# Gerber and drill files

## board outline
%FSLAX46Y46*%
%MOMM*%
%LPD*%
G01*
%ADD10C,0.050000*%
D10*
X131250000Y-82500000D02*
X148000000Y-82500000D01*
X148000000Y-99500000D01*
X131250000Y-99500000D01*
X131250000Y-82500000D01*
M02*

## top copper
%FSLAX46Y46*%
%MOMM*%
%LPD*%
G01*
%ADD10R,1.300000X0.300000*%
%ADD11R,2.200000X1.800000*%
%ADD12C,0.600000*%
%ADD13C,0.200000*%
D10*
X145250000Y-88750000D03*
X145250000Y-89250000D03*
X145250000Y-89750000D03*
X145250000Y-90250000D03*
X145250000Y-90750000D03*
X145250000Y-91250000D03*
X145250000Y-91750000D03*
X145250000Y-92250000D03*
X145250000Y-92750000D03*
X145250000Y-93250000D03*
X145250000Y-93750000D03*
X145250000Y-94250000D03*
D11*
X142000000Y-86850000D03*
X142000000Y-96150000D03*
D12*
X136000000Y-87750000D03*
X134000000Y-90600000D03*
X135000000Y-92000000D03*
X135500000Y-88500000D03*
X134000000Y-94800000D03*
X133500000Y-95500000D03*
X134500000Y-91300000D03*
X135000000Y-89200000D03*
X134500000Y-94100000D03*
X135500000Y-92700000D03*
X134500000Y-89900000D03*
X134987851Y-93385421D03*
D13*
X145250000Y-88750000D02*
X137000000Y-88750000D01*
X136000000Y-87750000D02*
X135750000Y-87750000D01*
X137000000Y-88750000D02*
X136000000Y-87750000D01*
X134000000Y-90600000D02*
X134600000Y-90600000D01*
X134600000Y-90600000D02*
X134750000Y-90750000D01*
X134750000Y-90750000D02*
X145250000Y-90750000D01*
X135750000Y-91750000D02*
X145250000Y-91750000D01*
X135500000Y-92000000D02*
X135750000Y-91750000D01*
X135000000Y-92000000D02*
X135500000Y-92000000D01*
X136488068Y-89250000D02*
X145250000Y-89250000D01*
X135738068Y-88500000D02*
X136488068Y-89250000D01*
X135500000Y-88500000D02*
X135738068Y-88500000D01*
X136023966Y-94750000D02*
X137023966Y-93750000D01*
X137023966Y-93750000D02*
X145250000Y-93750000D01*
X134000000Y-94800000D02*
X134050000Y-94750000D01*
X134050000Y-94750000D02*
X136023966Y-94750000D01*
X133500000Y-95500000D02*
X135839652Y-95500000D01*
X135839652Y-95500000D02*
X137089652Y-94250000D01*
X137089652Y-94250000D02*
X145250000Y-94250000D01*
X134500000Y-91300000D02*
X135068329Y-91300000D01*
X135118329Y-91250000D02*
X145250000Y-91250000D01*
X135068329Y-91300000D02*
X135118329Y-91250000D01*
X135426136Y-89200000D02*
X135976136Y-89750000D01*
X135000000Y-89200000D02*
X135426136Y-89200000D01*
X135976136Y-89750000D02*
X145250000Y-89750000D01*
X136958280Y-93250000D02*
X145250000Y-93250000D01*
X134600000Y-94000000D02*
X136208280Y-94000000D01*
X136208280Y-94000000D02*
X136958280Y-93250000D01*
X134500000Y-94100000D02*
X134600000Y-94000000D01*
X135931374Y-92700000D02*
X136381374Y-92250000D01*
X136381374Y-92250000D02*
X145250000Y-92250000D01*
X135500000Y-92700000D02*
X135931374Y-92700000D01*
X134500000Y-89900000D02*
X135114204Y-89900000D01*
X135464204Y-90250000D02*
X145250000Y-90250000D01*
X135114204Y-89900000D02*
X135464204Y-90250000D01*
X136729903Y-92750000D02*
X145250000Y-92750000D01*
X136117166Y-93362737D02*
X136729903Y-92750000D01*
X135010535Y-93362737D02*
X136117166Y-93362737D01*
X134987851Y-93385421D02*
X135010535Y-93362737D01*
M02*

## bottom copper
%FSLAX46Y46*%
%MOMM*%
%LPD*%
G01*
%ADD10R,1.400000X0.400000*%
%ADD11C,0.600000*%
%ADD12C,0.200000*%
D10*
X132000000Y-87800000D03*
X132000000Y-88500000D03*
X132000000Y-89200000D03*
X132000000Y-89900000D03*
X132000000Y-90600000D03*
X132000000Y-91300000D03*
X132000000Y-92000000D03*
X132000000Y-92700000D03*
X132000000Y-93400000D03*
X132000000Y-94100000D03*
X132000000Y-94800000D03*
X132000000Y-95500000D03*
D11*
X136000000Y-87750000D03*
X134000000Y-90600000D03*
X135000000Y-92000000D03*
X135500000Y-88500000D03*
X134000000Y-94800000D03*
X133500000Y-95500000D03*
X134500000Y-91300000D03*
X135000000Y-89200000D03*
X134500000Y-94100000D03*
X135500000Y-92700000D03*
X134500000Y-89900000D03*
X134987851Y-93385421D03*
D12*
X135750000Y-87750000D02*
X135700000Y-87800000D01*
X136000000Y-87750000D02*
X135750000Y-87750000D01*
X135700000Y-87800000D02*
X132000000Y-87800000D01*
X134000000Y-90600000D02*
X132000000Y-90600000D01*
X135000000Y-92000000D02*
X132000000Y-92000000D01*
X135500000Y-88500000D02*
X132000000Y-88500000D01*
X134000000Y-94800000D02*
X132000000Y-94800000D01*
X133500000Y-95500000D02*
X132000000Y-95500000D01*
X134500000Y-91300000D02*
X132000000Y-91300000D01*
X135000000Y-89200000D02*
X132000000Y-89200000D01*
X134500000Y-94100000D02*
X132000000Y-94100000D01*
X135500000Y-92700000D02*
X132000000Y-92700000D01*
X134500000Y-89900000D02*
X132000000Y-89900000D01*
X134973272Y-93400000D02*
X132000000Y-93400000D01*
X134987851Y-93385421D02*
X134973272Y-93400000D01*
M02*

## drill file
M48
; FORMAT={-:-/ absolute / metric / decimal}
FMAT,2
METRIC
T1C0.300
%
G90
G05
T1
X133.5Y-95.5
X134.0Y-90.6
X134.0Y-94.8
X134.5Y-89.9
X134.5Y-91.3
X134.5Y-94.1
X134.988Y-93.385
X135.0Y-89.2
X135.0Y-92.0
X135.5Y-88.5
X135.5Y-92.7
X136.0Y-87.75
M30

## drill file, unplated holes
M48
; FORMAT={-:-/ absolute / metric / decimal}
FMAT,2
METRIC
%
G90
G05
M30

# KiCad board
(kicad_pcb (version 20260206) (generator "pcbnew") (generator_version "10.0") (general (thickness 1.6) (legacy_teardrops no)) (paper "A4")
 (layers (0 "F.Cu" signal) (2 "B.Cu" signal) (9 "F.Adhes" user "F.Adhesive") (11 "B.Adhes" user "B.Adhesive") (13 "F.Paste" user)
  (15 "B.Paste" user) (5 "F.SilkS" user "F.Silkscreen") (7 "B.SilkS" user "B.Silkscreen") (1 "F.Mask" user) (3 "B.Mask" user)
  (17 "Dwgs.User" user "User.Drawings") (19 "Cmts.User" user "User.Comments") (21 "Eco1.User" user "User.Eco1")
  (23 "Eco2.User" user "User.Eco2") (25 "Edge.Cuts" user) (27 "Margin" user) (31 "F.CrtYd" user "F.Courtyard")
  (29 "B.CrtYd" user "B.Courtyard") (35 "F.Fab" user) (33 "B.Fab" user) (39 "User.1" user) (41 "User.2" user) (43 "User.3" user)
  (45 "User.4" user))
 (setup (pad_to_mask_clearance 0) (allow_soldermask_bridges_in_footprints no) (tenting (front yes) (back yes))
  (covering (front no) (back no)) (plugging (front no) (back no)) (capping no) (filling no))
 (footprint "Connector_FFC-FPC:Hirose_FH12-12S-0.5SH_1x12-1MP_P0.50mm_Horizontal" (layer "F.Cu") (at 143.4 91.5 -90)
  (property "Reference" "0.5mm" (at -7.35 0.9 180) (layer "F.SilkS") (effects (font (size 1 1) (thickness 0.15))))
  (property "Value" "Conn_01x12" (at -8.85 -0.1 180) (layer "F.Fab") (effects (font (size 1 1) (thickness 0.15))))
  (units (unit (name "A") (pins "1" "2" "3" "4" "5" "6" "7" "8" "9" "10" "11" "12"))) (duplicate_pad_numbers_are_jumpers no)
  (pad "1" smd rect (at -2.75 -1.85 270) (size 0.3 1.3) (layers "F.Cu" "F.Mask" "F.Paste") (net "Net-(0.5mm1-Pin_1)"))
  (pad "2" smd rect (at -2.25 -1.85 270) (size 0.3 1.3) (layers "F.Cu" "F.Mask" "F.Paste") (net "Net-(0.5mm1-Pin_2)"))
  (pad "3" smd rect (at -1.75 -1.85 270) (size 0.3 1.3) (layers "F.Cu" "F.Mask" "F.Paste") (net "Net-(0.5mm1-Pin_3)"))
  (pad "4" smd rect (at -1.25 -1.85 270) (size 0.3 1.3) (layers "F.Cu" "F.Mask" "F.Paste") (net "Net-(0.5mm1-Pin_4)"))
  (pad "5" smd rect (at -0.75 -1.85 270) (size 0.3 1.3) (layers "F.Cu" "F.Mask" "F.Paste") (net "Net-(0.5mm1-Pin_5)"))
  (pad "6" smd rect (at -0.25 -1.85 270) (size 0.3 1.3) (layers "F.Cu" "F.Mask" "F.Paste") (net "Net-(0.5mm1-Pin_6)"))
  (pad "7" smd rect (at 0.25 -1.85 270) (size 0.3 1.3) (layers "F.Cu" "F.Mask" "F.Paste") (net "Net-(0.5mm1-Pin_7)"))
  (pad "8" smd rect (at 0.75 -1.85 270) (size 0.3 1.3) (layers "F.Cu" "F.Mask" "F.Paste") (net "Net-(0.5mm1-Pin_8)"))
  (pad "9" smd rect (at 1.25 -1.85 270) (size 0.3 1.3) (layers "F.Cu" "F.Mask" "F.Paste") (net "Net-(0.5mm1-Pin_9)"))
  (pad "10" smd rect (at 1.75 -1.85 270) (size 0.3 1.3) (layers "F.Cu" "F.Mask" "F.Paste") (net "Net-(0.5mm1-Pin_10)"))
  (pad "11" smd rect (at 2.25 -1.85 270) (size 0.3 1.3) (layers "F.Cu" "F.Mask" "F.Paste") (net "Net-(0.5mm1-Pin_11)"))
  (pad "12" smd rect (at 2.75 -1.85 270) (size 0.3 1.3) (layers "F.Cu" "F.Mask" "F.Paste") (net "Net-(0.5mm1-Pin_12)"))
  (pad "MP" smd rect (at -4.65 1.4 270) (size 1.8 2.2) (layers "F.Cu" "F.Mask" "F.Paste"))
  (pad "MP" smd rect (at 4.65 1.4 270) (size 1.8 2.2) (layers "F.Cu" "F.Mask" "F.Paste")))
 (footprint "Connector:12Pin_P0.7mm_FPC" (layer "B.Cu") (at 132 91.65 -90)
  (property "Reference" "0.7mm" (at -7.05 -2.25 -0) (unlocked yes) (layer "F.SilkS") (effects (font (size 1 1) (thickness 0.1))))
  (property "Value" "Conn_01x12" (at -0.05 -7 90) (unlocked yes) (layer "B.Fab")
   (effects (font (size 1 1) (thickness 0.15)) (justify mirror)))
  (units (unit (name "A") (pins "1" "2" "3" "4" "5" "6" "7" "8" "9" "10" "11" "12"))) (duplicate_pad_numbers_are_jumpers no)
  (pad "1" connect rect (at -3.85 0 270) (size 0.4 1.4) (layers "B.Cu" "B.Mask") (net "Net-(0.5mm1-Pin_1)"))
  (pad "2" connect rect (at -3.15 0 270) (size 0.4 1.4) (layers "B.Cu" "B.Mask") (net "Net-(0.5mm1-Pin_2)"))
  (pad "3" connect rect (at -2.45 0 270) (size 0.4 1.4) (layers "B.Cu" "B.Mask") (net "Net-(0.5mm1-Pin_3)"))
  (pad "4" connect rect (at -1.75 0 270) (size 0.4 1.4) (layers "B.Cu" "B.Mask") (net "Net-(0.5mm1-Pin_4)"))
  (pad "5" connect rect (at -1.05 0 270) (size 0.4 1.4) (layers "B.Cu" "B.Mask") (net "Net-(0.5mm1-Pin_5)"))
  (pad "6" connect rect (at -0.35 0 270) (size 0.4 1.4) (layers "B.Cu" "B.Mask") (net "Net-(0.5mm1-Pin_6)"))
  (pad "7" connect rect (at 0.35 0 270) (size 0.4 1.4) (layers "B.Cu" "B.Mask") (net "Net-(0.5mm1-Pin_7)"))
  (pad "8" connect rect (at 1.05 0 270) (size 0.4 1.4) (layers "B.Cu" "B.Mask") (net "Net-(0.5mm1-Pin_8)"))
  (pad "9" connect rect (at 1.75 0 270) (size 0.4 1.4) (layers "B.Cu" "B.Mask") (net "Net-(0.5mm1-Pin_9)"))
  (pad "10" connect rect (at 2.45 0 270) (size 0.4 1.4) (layers "B.Cu" "B.Mask") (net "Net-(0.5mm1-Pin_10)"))
  (pad "11" connect rect (at 3.15 0 270) (size 0.4 1.4) (layers "B.Cu" "B.Mask") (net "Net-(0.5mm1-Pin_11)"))
  (pad "12" connect rect (at 3.85 0 270) (size 0.4 1.4) (layers "B.Cu" "B.Mask") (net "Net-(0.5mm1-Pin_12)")))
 (gr_rect (start 131.25 82.5) (end 148 99.5) (stroke (width 0.05) (type default)) (fill no) (layer "Edge.Cuts"))
 (segment (start 145.25 88.75) (end 137 88.75) (width 0.2) (layer "F.Cu") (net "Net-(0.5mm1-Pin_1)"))
 (segment (start 136 87.75) (end 135.75 87.75) (width 0.2) (layer "F.Cu") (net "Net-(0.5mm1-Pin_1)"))
 (segment (start 137 88.75) (end 136 87.75) (width 0.2) (layer "F.Cu") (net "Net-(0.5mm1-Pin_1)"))
 (via (at 136 87.75) (size 0.6) (drill 0.3) (layers "F.Cu" "B.Cu") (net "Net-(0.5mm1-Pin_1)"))
 (segment (start 135.75 87.75) (end 135.7 87.8) (width 0.2) (layer "B.Cu") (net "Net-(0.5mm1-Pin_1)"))
 (segment (start 136 87.75) (end 135.75 87.75) (width 0.2) (layer "B.Cu") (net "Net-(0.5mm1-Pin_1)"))
 (segment (start 135.7 87.8) (end 132 87.8) (width 0.2) (layer "B.Cu") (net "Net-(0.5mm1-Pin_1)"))
 (segment (start 134 90.6) (end 134.6 90.6) (width 0.2) (layer "F.Cu") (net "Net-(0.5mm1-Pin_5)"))
 (segment (start 134.6 90.6) (end 134.75 90.75) (width 0.2) (layer "F.Cu") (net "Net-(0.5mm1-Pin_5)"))
 (segment (start 134.75 90.75) (end 145.25 90.75) (width 0.2) (layer "F.Cu") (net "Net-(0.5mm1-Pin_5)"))
 (via (at 134 90.6) (size 0.6) (drill 0.3) (layers "F.Cu" "B.Cu") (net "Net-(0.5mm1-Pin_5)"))
 (segment (start 134 90.6) (end 132 90.6) (width 0.2) (layer "B.Cu") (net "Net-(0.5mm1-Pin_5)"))
 (segment (start 135.75 91.75) (end 145.25 91.75) (width 0.2) (layer "F.Cu") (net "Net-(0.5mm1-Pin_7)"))
 (segment (start 135.5 92) (end 135.75 91.75) (width 0.2) (layer "F.Cu") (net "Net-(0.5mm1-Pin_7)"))
 (segment (start 135 92) (end 135.5 92) (width 0.2) (layer "F.Cu") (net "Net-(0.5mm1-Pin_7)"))
 (via (at 135 92) (size 0.6) (drill 0.3) (layers "F.Cu" "B.Cu") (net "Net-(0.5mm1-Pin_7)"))
 (segment (start 135 92) (end 132 92) (width 0.2) (layer "B.Cu") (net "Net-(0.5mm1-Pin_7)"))
 (segment (start 136.488068 89.25) (end 145.25 89.25) (width 0.2) (layer "F.Cu") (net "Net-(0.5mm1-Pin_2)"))
 (segment (start 135.738068 88.5) (end 136.488068 89.25) (width 0.2) (layer "F.Cu") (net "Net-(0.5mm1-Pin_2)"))
 (segment (start 135.5 88.5) (end 135.738068 88.5) (width 0.2) (layer "F.Cu") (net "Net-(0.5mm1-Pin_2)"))
 (via (at 135.5 88.5) (size 0.6) (drill 0.3) (layers "F.Cu" "B.Cu") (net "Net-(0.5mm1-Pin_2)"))
 (segment (start 135.5 88.5) (end 132 88.5) (width 0.2) (layer "B.Cu") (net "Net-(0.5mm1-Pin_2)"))
 (segment (start 136.023966 94.75) (end 137.023966 93.75) (width 0.2) (layer "F.Cu") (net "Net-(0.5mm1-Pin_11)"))
 (segment (start 137.023966 93.75) (end 145.25 93.75) (width 0.2) (layer "F.Cu") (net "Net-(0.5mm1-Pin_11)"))
 (segment (start 134 94.8) (end 134.05 94.75) (width 0.2) (layer "F.Cu") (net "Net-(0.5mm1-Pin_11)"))
 (segment (start 134.05 94.75) (end 136.023966 94.75) (width 0.2) (layer "F.Cu") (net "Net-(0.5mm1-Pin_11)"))
 (via (at 134 94.8) (size 0.6) (drill 0.3) (layers "F.Cu" "B.Cu") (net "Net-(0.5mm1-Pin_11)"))
 (segment (start 134 94.8) (end 132 94.8) (width 0.2) (layer "B.Cu") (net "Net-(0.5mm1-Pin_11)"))
 (segment (start 133.5 95.5) (end 135.839652 95.5) (width 0.2) (layer "F.Cu") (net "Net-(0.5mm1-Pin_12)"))
 (segment (start 135.839652 95.5) (end 137.089652 94.25) (width 0.2) (layer "F.Cu") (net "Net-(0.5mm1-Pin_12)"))
 (segment (start 137.089652 94.25) (end 145.25 94.25) (width 0.2) (layer "F.Cu") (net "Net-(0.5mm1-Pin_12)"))
 (via (at 133.5 95.5) (size 0.6) (drill 0.3) (layers "F.Cu" "B.Cu") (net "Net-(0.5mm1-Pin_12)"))
 (segment (start 133.5 95.5) (end 132 95.5) (width 0.2) (layer "B.Cu") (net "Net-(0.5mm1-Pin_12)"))
 (segment (start 134.5 91.3) (end 135.068329 91.3) (width 0.2) (layer "F.Cu") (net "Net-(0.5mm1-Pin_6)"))
 (segment (start 135.118329 91.25) (end 145.25 91.25) (width 0.2) (layer "F.Cu") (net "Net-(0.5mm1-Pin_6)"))
 (segment (start 135.068329 91.3) (end 135.118329 91.25) (width 0.2) (layer "F.Cu") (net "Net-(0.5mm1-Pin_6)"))
 (via (at 134.5 91.3) (size 0.6) (drill 0.3) (layers "F.Cu" "B.Cu") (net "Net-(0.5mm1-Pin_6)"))
 (segment (start 134.5 91.3) (end 132 91.3) (width 0.2) (layer "B.Cu") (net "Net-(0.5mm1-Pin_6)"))
 (segment (start 135.426136 89.2) (end 135.976136 89.75) (width 0.2) (layer "F.Cu") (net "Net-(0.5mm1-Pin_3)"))
 (segment (start 135 89.2) (end 135.426136 89.2) (width 0.2) (layer "F.Cu") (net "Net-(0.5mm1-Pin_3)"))
 (segment (start 135.976136 89.75) (end 145.25 89.75) (width 0.2) (layer "F.Cu") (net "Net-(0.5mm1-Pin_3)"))
 (via (at 135 89.2) (size 0.6) (drill 0.3) (layers "F.Cu" "B.Cu") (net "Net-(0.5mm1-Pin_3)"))
 (segment (start 135 89.2) (end 132 89.2) (width 0.2) (layer "B.Cu") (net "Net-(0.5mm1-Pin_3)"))
 (segment (start 136.95828 93.25) (end 145.25 93.25) (width 0.2) (layer "F.Cu") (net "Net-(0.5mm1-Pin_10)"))
 (segment (start 134.6 94) (end 136.20828 94) (width 0.2) (layer "F.Cu") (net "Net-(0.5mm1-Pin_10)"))
 (segment (start 136.20828 94) (end 136.95828 93.25) (width 0.2) (layer "F.Cu") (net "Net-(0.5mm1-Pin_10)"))
 (segment (start 134.5 94.1) (end 134.6 94) (width 0.2) (layer "F.Cu") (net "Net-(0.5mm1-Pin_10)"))
 (via (at 134.5 94.1) (size 0.6) (drill 0.3) (layers "F.Cu" "B.Cu") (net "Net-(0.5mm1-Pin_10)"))
 (segment (start 134.5 94.1) (end 132 94.1) (width 0.2) (layer "B.Cu") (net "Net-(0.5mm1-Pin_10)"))
 (segment (start 135.931374 92.7) (end 136.381374 92.25) (width 0.2) (layer "F.Cu") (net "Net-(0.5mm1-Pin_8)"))
 (segment (start 136.381374 92.25) (end 145.25 92.25) (width 0.2) (layer "F.Cu") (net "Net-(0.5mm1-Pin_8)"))
 (segment (start 135.5 92.7) (end 135.931374 92.7) (width 0.2) (layer "F.Cu") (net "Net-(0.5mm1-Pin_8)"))
 (via (at 135.5 92.7) (size 0.6) (drill 0.3) (layers "F.Cu" "B.Cu") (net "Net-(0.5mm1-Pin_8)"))
 (segment (start 135.5 92.7) (end 132 92.7) (width 0.2) (layer "B.Cu") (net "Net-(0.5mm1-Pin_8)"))
 (segment (start 134.5 89.9) (end 135.114204 89.9) (width 0.2) (layer "F.Cu") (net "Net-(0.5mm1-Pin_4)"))
 (segment (start 135.464204 90.25) (end 145.25 90.25) (width 0.2) (layer "F.Cu") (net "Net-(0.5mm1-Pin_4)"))
 (segment (start 135.114204 89.9) (end 135.464204 90.25) (width 0.2) (layer "F.Cu") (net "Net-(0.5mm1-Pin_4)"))
 (via (at 134.5 89.9) (size 0.6) (drill 0.3) (layers "F.Cu" "B.Cu") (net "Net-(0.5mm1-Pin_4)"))
 (segment (start 134.5 89.9) (end 132 89.9) (width 0.2) (layer "B.Cu") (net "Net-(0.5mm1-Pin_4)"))
 (segment (start 136.729903 92.75) (end 145.25 92.75) (width 0.2) (layer "F.Cu") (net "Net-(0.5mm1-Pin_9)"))
 (segment (start 136.117166 93.362737) (end 136.729903 92.75) (width 0.2) (layer "F.Cu") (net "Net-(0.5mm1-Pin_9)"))
 (segment (start 135.010535 93.362737) (end 136.117166 93.362737) (width 0.2) (layer "F.Cu") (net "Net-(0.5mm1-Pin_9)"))
 (segment (start 134.987851 93.385421) (end 135.010535 93.362737) (width 0.2) (layer "F.Cu") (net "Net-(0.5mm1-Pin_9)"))
 (via (at 134.987851 93.385421) (size 0.6) (drill 0.3) (layers "F.Cu" "B.Cu") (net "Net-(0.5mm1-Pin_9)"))
 (segment (start 134.973272 93.4) (end 132 93.4) (width 0.2) (layer "B.Cu") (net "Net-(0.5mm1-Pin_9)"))
 (segment (start 134.987851 93.385421) (end 134.973272 93.4) (width 0.2) (layer "B.Cu") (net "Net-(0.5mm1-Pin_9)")))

